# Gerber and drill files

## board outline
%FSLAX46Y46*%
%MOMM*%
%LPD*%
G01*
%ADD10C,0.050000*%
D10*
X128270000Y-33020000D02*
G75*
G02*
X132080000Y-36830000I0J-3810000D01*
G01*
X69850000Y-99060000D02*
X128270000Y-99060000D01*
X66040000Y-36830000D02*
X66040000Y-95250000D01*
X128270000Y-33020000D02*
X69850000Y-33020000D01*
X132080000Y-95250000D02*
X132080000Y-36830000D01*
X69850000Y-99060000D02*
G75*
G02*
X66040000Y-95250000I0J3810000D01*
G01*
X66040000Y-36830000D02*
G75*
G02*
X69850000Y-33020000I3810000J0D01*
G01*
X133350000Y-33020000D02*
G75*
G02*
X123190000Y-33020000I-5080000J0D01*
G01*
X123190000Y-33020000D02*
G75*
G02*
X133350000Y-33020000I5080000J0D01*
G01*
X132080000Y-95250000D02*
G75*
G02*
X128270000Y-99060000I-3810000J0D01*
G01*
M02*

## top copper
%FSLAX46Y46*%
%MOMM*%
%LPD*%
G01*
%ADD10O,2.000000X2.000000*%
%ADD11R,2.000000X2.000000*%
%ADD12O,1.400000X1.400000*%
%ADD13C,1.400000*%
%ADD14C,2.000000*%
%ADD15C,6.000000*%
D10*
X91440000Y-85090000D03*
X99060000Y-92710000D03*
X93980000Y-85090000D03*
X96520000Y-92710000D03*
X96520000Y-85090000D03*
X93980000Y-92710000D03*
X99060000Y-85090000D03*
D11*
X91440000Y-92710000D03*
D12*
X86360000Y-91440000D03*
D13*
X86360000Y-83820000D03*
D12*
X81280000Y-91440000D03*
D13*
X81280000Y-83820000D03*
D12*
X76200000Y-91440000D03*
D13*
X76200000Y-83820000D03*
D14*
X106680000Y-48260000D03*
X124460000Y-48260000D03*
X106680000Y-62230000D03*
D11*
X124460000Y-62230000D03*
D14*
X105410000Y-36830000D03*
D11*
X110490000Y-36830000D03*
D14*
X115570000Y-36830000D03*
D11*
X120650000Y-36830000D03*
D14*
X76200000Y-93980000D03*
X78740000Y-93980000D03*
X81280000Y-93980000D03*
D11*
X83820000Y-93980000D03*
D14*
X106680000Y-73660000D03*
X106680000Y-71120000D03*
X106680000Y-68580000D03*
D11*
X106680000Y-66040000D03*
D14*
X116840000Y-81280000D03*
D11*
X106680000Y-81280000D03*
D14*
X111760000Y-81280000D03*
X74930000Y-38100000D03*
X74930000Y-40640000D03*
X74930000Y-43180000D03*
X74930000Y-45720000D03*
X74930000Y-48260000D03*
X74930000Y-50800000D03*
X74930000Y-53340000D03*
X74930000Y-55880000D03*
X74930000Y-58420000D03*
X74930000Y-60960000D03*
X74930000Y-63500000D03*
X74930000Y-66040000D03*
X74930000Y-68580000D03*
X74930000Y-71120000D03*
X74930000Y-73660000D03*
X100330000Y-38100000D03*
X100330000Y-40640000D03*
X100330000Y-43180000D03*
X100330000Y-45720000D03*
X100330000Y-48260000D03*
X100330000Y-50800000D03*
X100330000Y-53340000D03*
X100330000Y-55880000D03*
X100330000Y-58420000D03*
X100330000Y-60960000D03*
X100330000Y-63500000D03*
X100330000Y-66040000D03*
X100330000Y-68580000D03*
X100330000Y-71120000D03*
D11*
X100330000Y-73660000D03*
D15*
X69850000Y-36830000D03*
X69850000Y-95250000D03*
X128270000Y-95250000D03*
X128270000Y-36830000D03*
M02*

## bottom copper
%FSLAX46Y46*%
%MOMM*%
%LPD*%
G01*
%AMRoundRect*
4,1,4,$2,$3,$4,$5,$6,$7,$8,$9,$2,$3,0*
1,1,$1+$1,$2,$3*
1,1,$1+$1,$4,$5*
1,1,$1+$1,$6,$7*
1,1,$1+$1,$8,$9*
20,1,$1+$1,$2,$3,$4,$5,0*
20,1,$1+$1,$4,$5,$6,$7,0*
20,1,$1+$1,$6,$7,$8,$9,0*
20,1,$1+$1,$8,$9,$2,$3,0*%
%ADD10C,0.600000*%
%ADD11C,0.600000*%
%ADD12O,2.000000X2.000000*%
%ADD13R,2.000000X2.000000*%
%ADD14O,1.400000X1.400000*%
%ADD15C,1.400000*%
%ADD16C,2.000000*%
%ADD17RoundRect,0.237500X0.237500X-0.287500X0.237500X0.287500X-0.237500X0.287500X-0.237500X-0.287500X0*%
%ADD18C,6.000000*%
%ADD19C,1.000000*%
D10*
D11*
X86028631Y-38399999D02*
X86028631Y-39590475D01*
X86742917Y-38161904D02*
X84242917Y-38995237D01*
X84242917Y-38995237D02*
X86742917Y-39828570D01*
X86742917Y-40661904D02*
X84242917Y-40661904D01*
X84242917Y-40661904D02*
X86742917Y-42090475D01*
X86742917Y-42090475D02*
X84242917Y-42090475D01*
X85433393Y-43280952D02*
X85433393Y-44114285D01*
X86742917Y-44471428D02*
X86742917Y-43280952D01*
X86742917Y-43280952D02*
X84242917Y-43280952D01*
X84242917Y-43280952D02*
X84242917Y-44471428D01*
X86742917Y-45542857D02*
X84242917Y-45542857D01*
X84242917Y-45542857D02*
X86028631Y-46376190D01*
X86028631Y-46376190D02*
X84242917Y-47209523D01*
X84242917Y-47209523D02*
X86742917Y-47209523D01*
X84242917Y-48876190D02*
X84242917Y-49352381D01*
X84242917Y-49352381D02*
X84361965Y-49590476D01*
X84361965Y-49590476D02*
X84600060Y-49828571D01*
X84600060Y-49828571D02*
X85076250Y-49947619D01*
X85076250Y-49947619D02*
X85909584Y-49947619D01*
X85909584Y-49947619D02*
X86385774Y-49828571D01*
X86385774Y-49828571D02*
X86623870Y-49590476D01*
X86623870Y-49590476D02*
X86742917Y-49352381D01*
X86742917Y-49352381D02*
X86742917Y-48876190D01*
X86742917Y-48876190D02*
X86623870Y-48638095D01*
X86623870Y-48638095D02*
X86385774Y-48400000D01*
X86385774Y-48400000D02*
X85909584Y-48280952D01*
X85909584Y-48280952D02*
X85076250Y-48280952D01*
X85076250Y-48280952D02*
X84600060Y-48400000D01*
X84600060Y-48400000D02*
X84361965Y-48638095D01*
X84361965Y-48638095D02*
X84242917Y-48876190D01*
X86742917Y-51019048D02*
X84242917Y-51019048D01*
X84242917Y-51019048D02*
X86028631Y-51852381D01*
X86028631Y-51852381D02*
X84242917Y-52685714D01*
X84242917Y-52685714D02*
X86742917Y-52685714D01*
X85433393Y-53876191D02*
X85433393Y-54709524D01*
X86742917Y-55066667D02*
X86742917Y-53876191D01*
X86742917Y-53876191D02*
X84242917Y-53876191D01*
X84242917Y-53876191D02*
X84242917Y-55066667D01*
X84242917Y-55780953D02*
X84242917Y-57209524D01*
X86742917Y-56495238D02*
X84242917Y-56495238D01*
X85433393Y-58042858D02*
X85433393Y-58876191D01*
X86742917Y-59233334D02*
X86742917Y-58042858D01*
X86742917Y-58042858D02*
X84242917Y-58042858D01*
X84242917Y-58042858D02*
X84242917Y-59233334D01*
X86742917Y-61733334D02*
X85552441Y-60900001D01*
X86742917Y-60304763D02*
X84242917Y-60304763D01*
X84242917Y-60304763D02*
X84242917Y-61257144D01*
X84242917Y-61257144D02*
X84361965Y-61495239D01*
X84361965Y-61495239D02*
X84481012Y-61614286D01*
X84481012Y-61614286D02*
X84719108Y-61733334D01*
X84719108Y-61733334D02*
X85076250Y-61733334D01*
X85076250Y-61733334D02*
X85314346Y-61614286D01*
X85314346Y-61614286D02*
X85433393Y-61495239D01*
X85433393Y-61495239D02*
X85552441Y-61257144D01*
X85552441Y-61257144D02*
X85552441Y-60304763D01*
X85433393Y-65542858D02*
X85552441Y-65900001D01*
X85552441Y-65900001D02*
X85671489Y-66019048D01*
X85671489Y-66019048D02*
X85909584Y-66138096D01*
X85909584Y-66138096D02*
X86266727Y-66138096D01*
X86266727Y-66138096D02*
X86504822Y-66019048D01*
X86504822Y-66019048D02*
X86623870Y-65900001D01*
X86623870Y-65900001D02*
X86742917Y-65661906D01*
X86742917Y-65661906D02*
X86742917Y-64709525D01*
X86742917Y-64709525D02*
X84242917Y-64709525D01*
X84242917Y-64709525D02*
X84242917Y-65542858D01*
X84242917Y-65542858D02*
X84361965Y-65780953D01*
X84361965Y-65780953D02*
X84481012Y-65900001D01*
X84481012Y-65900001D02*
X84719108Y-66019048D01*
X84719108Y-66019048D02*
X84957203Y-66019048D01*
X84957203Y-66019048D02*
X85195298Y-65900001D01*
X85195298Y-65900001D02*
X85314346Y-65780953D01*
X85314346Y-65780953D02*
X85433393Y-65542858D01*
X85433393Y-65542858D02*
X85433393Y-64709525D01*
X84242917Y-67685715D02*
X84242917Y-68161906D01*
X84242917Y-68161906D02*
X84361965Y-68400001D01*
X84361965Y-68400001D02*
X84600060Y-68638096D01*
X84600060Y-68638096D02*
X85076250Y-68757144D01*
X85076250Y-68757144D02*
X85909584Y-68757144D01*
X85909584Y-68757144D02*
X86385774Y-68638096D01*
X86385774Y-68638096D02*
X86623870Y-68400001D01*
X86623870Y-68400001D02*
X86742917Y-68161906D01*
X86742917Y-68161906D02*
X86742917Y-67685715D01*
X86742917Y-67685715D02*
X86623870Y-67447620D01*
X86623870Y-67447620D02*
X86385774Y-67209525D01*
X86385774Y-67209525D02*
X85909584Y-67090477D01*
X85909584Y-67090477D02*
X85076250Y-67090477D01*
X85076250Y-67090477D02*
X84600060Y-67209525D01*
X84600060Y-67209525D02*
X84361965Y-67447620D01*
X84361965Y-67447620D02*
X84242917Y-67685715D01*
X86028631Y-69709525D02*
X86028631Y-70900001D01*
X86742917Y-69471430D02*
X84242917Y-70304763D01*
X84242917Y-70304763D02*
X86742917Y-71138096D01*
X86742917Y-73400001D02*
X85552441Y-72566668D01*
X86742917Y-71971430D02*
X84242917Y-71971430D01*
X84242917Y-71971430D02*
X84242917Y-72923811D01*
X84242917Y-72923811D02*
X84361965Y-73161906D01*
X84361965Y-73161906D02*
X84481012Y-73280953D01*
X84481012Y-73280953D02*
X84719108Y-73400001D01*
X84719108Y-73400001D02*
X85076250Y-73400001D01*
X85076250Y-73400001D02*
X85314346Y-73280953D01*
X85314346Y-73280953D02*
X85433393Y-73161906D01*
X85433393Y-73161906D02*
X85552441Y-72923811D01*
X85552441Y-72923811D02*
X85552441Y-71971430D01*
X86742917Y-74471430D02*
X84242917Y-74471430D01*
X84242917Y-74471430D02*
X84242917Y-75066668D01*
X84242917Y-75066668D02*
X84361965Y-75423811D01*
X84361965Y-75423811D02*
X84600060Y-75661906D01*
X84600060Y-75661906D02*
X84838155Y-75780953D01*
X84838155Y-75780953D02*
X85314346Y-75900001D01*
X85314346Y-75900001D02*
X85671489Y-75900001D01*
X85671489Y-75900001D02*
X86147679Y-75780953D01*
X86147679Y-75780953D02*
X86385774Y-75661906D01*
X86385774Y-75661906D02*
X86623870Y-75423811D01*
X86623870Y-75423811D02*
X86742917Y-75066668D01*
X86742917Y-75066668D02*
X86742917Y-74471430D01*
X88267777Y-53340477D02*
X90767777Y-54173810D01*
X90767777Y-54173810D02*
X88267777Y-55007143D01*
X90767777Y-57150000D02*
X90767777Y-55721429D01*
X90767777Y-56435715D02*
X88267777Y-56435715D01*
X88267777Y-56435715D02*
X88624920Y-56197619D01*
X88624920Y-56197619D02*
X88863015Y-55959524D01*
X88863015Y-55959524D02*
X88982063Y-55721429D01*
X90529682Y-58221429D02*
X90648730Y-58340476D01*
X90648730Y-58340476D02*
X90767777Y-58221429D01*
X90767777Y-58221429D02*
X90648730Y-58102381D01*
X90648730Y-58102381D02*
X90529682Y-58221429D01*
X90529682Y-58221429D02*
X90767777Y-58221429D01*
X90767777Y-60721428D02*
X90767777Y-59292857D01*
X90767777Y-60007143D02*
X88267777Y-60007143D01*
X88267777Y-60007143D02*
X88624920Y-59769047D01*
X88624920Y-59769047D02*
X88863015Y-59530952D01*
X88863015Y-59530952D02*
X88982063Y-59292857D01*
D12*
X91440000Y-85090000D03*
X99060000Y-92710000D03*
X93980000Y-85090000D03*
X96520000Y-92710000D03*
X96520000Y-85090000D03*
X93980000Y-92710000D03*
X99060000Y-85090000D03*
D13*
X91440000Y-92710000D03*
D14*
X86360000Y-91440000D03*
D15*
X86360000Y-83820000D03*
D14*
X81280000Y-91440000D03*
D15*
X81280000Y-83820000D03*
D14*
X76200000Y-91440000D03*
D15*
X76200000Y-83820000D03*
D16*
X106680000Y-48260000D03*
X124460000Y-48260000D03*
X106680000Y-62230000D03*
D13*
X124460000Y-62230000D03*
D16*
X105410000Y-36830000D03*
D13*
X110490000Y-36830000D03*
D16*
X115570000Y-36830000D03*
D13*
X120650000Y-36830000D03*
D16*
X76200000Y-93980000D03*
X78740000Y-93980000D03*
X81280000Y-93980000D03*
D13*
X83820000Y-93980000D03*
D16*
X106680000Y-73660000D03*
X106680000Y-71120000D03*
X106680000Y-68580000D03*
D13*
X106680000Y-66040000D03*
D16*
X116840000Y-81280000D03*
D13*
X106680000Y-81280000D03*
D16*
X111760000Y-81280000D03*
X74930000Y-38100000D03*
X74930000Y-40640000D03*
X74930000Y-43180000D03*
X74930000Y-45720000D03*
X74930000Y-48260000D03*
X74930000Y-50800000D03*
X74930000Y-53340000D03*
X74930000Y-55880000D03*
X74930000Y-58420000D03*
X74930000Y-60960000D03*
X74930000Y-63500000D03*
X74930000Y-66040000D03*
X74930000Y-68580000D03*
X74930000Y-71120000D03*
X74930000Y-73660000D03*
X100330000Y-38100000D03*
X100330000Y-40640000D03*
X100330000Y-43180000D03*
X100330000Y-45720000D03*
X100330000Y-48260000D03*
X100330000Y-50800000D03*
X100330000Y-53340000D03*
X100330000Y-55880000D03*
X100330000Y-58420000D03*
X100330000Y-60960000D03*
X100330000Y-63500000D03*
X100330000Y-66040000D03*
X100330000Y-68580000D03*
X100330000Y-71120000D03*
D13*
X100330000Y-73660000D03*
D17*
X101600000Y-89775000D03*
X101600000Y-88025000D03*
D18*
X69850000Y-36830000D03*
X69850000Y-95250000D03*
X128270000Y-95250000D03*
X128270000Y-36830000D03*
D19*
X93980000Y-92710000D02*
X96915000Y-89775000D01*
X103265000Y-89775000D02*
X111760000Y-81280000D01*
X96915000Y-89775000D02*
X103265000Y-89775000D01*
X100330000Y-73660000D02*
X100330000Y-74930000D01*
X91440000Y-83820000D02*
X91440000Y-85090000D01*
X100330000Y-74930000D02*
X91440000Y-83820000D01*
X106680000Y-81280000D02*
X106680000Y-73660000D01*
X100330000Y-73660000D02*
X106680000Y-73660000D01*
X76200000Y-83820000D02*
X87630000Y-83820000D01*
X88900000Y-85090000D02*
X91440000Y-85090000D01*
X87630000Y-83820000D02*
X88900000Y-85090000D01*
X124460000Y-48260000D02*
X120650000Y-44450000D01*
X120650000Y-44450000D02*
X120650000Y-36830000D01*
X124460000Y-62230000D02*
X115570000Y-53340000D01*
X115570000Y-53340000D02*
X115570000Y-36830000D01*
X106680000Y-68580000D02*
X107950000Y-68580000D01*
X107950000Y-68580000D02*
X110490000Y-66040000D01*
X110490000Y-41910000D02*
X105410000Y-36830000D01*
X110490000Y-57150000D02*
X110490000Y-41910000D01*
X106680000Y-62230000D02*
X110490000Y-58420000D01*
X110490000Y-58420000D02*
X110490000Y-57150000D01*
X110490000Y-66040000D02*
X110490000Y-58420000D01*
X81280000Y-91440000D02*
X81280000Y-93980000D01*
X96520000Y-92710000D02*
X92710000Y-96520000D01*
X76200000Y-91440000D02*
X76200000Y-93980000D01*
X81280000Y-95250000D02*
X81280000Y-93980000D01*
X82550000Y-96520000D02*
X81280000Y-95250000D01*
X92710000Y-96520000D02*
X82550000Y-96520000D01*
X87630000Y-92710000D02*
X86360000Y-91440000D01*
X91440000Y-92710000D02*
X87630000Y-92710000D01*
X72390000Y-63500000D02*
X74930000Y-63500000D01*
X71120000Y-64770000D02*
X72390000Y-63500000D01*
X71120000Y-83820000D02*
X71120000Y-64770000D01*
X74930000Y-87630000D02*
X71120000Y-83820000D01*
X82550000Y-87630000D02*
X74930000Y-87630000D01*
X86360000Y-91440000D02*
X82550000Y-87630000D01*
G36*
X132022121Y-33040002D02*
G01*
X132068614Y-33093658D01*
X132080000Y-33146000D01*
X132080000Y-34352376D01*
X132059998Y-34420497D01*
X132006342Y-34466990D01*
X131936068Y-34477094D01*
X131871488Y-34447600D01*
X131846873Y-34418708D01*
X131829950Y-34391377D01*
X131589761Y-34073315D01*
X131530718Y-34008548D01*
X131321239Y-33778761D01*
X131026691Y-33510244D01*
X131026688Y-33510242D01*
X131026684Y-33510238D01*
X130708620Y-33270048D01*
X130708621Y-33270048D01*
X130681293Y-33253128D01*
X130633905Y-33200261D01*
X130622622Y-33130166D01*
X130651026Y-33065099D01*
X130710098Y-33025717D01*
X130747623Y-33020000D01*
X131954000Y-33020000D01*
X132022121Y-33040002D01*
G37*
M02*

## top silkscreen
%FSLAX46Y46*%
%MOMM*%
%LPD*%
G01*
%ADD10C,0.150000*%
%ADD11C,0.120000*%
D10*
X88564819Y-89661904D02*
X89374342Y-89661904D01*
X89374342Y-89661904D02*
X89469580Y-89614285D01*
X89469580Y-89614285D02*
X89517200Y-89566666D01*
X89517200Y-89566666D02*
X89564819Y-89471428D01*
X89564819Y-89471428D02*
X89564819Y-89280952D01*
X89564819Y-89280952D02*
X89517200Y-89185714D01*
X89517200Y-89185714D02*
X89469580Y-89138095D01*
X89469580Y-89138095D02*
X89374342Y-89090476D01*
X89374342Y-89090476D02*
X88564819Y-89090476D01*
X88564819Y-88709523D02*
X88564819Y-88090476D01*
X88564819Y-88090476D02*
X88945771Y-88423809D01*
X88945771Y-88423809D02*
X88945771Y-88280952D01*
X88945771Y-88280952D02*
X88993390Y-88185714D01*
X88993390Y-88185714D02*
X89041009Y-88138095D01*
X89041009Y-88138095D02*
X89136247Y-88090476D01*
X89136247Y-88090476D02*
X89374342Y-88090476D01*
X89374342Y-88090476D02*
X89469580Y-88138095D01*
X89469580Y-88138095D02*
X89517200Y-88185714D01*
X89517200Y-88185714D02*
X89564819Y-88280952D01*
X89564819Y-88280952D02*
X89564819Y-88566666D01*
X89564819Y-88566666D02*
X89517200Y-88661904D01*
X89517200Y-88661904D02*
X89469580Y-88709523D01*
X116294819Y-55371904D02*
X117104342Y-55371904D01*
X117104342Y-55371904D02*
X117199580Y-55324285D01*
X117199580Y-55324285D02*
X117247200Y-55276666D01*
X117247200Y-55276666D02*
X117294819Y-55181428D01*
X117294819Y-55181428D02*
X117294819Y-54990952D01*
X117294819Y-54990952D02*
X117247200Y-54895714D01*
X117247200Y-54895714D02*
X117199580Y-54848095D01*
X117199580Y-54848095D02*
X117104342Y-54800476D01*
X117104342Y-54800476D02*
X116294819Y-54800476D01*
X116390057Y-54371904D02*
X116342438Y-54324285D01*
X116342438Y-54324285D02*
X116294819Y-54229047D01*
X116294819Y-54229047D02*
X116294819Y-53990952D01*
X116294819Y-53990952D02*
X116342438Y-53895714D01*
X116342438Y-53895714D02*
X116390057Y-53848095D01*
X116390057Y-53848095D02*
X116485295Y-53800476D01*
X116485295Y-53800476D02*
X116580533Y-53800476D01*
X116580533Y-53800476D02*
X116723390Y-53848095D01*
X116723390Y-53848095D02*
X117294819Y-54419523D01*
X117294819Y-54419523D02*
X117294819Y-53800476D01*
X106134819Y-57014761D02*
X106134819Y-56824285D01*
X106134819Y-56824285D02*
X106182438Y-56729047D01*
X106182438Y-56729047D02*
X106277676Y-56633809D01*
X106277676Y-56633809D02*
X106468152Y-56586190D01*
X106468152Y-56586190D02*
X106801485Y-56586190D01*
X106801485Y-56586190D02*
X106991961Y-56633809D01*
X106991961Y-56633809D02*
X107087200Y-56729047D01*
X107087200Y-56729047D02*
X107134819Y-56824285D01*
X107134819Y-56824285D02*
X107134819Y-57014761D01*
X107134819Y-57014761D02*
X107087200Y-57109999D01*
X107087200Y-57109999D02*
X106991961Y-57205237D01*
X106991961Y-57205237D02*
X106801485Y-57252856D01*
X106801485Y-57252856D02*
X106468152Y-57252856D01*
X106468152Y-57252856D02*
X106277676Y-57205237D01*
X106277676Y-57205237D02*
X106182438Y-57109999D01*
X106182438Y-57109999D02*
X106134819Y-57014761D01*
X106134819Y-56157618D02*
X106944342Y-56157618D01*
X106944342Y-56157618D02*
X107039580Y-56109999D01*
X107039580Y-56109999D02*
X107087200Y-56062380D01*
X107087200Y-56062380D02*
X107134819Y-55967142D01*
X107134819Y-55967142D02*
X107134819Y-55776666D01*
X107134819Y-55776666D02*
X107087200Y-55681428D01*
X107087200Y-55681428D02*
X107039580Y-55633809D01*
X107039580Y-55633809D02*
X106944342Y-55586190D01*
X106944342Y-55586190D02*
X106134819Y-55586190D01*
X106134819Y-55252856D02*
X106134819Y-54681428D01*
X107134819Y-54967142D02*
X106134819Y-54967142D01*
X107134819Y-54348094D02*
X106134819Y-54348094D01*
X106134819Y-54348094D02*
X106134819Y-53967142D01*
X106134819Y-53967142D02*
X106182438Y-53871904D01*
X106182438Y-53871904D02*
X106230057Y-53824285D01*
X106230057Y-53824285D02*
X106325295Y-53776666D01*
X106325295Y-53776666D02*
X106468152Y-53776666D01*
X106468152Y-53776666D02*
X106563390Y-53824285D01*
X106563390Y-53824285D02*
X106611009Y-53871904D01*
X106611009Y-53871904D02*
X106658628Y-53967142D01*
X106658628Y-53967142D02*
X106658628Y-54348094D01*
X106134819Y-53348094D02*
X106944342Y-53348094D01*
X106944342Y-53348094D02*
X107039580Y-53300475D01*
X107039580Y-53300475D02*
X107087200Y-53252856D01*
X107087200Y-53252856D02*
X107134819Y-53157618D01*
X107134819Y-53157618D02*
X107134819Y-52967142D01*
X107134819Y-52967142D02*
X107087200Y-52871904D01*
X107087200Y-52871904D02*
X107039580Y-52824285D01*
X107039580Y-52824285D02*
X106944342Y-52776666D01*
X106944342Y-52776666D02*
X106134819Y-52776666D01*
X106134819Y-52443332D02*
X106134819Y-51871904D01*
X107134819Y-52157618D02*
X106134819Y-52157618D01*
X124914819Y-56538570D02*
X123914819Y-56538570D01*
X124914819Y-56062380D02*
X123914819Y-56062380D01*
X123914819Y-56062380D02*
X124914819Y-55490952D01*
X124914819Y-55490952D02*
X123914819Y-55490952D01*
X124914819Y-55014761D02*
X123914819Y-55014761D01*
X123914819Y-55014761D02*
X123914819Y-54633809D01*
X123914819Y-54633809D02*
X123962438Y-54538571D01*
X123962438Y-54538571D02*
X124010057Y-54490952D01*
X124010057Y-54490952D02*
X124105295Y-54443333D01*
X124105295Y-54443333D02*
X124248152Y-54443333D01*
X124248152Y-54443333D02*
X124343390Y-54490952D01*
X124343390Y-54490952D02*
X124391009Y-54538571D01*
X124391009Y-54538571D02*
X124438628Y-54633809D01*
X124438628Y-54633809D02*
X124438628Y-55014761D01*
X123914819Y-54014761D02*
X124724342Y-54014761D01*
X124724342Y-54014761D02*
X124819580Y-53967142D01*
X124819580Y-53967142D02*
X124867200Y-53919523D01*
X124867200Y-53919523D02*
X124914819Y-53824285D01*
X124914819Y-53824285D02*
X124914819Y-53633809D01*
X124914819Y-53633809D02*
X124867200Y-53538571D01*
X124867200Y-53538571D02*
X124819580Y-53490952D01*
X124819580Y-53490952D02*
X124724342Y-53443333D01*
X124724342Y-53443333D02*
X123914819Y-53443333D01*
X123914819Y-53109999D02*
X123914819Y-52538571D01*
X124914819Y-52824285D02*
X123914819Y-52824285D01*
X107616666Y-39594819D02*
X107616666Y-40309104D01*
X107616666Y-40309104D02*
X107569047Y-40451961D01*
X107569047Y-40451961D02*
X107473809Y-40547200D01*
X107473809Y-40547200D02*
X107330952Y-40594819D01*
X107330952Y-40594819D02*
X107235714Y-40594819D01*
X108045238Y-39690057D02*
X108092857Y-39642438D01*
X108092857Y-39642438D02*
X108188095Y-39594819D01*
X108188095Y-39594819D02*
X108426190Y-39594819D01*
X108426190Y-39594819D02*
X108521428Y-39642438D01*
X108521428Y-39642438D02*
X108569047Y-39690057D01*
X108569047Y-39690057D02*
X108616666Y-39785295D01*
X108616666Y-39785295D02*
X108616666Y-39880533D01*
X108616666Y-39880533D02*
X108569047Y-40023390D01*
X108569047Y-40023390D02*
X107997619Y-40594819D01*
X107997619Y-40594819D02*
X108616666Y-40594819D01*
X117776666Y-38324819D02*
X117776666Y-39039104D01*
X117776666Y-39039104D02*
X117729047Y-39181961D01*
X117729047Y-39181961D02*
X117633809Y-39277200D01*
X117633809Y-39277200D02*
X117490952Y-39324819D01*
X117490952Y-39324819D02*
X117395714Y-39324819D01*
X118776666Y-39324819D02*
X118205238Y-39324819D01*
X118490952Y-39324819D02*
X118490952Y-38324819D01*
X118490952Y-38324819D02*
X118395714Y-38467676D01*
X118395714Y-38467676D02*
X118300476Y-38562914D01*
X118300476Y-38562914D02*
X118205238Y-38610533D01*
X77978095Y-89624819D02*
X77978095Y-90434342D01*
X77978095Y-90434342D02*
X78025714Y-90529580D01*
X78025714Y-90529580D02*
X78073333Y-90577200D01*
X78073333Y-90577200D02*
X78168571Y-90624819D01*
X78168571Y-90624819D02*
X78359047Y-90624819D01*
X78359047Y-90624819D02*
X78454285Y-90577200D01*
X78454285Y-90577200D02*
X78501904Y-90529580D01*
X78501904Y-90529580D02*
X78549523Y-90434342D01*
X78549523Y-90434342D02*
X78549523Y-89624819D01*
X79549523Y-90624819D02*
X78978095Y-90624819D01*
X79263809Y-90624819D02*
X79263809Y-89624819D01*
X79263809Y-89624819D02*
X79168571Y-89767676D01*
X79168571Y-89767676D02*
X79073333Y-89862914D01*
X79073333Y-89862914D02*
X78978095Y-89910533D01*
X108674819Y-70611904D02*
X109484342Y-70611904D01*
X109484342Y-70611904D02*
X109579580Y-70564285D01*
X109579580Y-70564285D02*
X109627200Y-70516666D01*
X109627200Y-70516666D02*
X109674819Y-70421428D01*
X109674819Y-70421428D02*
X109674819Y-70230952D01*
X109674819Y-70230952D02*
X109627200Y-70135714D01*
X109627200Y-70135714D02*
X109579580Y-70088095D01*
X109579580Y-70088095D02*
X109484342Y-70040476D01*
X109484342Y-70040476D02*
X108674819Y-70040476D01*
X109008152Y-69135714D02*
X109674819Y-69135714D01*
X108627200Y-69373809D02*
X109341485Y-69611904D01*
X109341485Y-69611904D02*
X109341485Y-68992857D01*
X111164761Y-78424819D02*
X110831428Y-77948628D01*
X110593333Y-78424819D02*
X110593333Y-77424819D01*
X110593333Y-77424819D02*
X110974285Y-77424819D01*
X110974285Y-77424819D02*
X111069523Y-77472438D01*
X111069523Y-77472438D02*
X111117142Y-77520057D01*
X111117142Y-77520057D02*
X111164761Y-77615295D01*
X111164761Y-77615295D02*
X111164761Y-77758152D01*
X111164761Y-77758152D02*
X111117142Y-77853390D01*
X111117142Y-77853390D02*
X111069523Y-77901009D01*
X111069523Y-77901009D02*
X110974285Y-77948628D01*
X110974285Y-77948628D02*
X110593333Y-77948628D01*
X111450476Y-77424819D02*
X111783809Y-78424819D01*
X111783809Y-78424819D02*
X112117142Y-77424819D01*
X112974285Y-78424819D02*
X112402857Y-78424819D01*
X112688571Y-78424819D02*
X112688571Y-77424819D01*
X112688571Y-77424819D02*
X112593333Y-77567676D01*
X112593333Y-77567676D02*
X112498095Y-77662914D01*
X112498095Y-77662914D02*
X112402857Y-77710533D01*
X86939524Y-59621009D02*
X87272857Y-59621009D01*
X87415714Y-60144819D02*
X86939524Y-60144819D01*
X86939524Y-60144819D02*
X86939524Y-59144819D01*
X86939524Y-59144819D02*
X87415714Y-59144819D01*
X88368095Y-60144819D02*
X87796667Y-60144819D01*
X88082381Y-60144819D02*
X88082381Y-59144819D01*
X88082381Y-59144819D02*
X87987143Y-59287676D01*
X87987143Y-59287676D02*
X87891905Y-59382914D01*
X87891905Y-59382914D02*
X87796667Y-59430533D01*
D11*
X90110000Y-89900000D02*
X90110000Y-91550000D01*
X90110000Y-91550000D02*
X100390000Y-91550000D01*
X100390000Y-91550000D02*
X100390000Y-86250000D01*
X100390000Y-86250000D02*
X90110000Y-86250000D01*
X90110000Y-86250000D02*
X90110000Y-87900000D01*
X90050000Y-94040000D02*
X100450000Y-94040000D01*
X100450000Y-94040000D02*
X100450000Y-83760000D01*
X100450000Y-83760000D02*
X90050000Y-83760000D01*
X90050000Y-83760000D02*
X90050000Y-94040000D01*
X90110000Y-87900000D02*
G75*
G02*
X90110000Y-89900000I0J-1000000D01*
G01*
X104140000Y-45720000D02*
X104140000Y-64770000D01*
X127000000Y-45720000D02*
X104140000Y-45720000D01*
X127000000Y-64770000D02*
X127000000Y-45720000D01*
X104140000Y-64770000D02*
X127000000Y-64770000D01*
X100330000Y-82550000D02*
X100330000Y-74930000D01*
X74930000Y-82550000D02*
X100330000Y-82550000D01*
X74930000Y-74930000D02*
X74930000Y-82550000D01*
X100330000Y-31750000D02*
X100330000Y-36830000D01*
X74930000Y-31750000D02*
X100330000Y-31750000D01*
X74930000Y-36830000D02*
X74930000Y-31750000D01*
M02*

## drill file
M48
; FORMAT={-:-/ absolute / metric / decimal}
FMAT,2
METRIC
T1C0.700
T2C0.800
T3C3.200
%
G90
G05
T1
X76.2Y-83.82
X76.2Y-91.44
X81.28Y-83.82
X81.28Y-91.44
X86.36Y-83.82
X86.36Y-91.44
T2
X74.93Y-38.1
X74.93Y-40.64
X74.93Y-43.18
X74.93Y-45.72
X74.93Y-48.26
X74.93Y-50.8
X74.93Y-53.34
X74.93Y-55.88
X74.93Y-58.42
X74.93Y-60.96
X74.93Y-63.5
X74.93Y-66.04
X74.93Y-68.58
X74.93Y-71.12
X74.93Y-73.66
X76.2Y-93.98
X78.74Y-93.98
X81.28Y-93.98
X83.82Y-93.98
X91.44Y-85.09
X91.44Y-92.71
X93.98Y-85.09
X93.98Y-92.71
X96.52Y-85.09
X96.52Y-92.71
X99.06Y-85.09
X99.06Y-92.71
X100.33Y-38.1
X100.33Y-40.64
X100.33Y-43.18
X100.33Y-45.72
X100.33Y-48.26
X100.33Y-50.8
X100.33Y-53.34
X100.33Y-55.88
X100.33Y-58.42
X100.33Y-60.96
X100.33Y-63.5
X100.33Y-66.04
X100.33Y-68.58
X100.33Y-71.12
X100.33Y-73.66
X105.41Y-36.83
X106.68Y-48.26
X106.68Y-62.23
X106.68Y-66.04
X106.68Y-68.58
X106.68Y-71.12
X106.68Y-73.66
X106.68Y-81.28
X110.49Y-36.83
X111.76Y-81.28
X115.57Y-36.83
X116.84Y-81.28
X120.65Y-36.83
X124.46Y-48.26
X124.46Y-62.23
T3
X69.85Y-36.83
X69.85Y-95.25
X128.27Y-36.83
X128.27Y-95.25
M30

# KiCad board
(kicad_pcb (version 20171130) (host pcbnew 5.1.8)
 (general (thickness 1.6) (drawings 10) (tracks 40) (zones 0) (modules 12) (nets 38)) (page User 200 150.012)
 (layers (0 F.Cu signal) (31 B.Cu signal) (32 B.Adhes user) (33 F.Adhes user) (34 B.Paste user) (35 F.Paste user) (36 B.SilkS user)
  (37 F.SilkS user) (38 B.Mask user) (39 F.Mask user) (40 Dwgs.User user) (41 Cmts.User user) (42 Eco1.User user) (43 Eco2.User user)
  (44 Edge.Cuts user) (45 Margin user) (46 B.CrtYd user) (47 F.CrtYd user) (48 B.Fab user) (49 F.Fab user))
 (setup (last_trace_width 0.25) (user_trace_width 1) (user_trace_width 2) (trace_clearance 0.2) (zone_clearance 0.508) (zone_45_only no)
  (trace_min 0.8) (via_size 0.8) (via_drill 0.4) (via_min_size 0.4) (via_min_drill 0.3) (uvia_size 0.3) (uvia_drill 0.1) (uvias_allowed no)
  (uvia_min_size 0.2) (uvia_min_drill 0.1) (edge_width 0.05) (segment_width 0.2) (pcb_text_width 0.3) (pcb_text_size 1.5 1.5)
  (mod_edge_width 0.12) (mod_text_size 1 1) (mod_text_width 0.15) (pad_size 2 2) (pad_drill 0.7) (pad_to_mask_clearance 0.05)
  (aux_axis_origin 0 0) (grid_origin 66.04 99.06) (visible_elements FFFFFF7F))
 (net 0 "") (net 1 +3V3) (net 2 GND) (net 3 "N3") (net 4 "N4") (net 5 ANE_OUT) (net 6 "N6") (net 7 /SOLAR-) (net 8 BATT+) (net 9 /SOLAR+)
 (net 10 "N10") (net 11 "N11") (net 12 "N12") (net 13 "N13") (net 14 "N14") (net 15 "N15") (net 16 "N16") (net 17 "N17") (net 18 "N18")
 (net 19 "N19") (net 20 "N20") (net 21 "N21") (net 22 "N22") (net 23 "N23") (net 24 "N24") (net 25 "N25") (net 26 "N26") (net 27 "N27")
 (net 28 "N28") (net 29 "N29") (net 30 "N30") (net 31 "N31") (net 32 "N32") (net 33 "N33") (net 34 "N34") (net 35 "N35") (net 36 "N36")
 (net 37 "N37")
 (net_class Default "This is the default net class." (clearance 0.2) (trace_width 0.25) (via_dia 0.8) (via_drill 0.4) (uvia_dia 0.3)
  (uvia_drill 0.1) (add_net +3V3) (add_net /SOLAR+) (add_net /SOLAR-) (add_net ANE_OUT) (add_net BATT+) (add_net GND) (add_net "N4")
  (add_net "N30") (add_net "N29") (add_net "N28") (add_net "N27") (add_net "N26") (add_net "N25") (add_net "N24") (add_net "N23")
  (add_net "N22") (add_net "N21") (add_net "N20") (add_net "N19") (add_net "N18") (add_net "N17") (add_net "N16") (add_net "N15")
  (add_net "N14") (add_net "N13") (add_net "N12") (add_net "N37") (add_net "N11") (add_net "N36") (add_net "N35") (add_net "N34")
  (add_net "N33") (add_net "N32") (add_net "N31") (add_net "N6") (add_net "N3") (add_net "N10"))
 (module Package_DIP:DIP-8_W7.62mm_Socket (layer F.Cu) (at 91.44 92.71 90)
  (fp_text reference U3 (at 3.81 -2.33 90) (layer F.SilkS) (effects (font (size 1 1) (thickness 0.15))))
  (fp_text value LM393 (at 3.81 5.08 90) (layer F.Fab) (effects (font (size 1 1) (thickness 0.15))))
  (fp_line (start 2.81 -1.33) (end 1.16 -1.33) (layer F.SilkS) (width 0.12))
  (fp_line (start 1.16 -1.33) (end 1.16 8.95) (layer F.SilkS) (width 0.12))
  (fp_line (start 1.16 8.95) (end 6.46 8.95) (layer F.SilkS) (width 0.12))
  (fp_line (start 6.46 8.95) (end 6.46 -1.33) (layer F.SilkS) (width 0.12))
  (fp_line (start 6.46 -1.33) (end 4.81 -1.33) (layer F.SilkS) (width 0.12))
  (fp_line (start -1.33 -1.39) (end -1.33 9.01) (layer F.SilkS) (width 0.12))
  (fp_line (start -1.33 9.01) (end 8.95 9.01) (layer F.SilkS) (width 0.12))
  (fp_line (start 8.95 9.01) (end 8.95 -1.39) (layer F.SilkS) (width 0.12))
  (fp_line (start 8.95 -1.39) (end -1.33 -1.39) (layer F.SilkS) (width 0.12))
  (fp_arc (start 3.81 -1.33) (end 2.81 -1.33) (angle -180) (layer F.SilkS) (width 0.12))
  (pad 8 thru_hole oval (at 7.62 0 90) (size 2 2) (drill 0.8) (layers *.Cu *.Mask) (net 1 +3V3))
  (pad 4 thru_hole oval (at 0 7.62 90) (size 2 2) (drill 0.8) (layers *.Cu *.Mask) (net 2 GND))
  (pad 7 thru_hole oval (at 7.62 2.54 90) (size 2 2) (drill 0.8) (layers *.Cu *.Mask))
  (pad 3 thru_hole oval (at 0 5.08 90) (size 2 2) (drill 0.8) (layers *.Cu *.Mask) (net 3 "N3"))
  (pad 6 thru_hole oval (at 7.62 5.08 90) (size 2 2) (drill 0.8) (layers *.Cu *.Mask))
  (pad 2 thru_hole oval (at 0 2.54 90) (size 2 2) (drill 0.8) (layers *.Cu *.Mask) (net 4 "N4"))
  (pad 5 thru_hole oval (at 7.62 7.62 90) (size 2 2) (drill 0.8) (layers *.Cu *.Mask))
  (pad 1 thru_hole rect (at 0 0 90) (size 2 2) (drill 0.8) (layers *.Cu *.Mask) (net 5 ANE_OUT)))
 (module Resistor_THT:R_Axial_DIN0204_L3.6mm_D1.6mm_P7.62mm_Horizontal (layer B.Cu) (at 86.36 83.82 270)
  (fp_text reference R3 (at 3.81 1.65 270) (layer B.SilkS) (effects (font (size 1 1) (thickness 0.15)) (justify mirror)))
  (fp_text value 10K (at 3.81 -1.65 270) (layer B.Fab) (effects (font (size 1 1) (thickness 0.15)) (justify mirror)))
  (pad 2 thru_hole oval (at 7.62 0 270) (size 1.4 1.4) (drill 0.7) (layers *.Cu *.Mask) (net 5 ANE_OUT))
  (pad 1 thru_hole circle (at 0 0 270) (size 1.4 1.4) (drill 0.7) (layers *.Cu *.Mask) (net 1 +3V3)))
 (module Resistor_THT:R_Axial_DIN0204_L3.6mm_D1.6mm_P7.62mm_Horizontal (layer B.Cu) (at 81.28 83.82 270)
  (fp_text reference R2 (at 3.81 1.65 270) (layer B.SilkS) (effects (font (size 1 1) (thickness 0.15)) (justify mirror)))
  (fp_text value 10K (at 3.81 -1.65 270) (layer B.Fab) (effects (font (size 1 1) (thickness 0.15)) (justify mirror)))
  (pad 2 thru_hole oval (at 7.62 0 270) (size 1.4 1.4) (drill 0.7) (layers *.Cu *.Mask) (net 3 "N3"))
  (pad 1 thru_hole circle (at 0 0 270) (size 1.4 1.4) (drill 0.7) (layers *.Cu *.Mask) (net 1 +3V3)))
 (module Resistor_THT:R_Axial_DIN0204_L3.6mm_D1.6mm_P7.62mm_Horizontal (layer B.Cu) (at 76.2 83.82 270)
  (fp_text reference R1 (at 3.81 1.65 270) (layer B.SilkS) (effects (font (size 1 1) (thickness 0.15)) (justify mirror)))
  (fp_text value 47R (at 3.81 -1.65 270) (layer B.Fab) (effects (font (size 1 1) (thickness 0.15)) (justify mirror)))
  (pad 2 thru_hole oval (at 7.62 0 270) (size 1.4 1.4) (drill 0.7) (layers *.Cu *.Mask) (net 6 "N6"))
  (pad 1 thru_hole circle (at 0 0 270) (size 1.4 1.4) (drill 0.7) (layers *.Cu *.Mask) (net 1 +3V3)))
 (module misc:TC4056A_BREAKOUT (layer F.Cu) (at 115.57 54.61 90)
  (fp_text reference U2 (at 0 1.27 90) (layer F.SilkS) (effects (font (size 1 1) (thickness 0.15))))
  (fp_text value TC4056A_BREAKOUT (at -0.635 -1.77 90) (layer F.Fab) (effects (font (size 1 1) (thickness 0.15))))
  (fp_line (start 8.89 -11.43) (end -10.16 -11.43) (layer F.SilkS) (width 0.12))
  (fp_line (start 8.89 11.43) (end 8.89 -11.43) (layer F.SilkS) (width 0.12))
  (fp_line (start -10.16 11.43) (end 8.89 11.43) (layer F.SilkS) (width 0.12))
  (fp_line (start -10.16 -11.43) (end -10.16 11.43) (layer F.SilkS) (width 0.12))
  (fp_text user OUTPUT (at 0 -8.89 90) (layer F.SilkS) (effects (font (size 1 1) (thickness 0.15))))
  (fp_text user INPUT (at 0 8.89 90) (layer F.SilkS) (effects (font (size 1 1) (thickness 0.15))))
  (pad 3 thru_hole circle (at 6.35 -8.89 90) (size 2 2) (drill 0.8) (layers *.Cu *.Mask) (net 2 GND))
  (pad 2 thru_hole circle (at 6.35 8.89 90) (size 2 2) (drill 0.8) (layers *.Cu *.Mask) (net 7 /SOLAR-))
  (pad 4 thru_hole circle (at -7.62 -8.89 90) (size 2 2) (drill 0.8) (layers *.Cu *.Mask) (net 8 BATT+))
  (pad 1 thru_hole rect (at -7.62 8.89 90) (size 2 2) (drill 0.8) (layers *.Cu *.Mask) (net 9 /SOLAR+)))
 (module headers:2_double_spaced (layer F.Cu) (at 107.95 36.83 180)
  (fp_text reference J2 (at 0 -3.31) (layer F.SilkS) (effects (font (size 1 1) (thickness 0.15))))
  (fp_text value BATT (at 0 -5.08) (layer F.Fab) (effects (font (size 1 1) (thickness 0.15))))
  (pad 2 thru_hole circle (at 2.54 0 180) (size 2 2) (drill 0.8) (layers *.Cu *.Mask) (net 8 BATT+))
  (pad 1 thru_hole rect (at -2.54 0 180) (size 2 2) (drill 0.8) (layers *.Cu *.Mask) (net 2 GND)))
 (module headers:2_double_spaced (layer F.Cu) (at 118.11 36.83 180)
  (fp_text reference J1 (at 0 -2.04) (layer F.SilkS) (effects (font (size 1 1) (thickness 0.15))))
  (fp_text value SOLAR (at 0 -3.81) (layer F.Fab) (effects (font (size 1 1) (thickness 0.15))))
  (pad 2 thru_hole circle (at 2.54 0 180) (size 2 2) (drill 0.8) (layers *.Cu *.Mask) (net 9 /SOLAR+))
  (pad 1 thru_hole rect (at -2.54 0 180) (size 2 2) (drill 0.8) (layers *.Cu *.Mask) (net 7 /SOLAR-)))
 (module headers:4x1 (layer F.Cu) (at 80.01 93.98 180)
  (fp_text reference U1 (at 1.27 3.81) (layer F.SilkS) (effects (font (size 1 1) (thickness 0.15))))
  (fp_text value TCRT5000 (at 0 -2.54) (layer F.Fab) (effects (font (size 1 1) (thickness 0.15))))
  (pad 4 thru_hole circle (at 3.81 0 180) (size 2 2) (drill 0.8) (layers *.Cu *.Mask) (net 6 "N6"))
  (pad 3 thru_hole circle (at 1.27 0 180) (size 2 2) (drill 0.8) (layers *.Cu *.Mask) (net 2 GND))
  (pad 2 thru_hole circle (at -1.27 0 180) (size 2 2) (drill 0.8) (layers *.Cu *.Mask) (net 3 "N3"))
  (pad 1 thru_hole rect (at -3.81 0 180) (size 2 2) (drill 0.8) (layers *.Cu *.Mask) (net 2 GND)))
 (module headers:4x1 (layer F.Cu) (at 106.68 69.85 270)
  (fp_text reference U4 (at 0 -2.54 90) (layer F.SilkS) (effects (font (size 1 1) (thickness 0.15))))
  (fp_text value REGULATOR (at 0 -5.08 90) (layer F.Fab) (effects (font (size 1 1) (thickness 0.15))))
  (pad 4 thru_hole circle (at 3.81 0 270) (size 2 2) (drill 0.8) (layers *.Cu *.Mask) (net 1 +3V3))
  (pad 3 thru_hole circle (at 1.27 0 270) (size 2 2) (drill 0.8) (layers *.Cu *.Mask) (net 2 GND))
  (pad 2 thru_hole circle (at -1.27 0 270) (size 2 2) (drill 0.8) (layers *.Cu *.Mask) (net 8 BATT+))
  (pad 1 thru_hole rect (at -3.81 0 270) (size 2 2) (drill 0.8) (layers *.Cu *.Mask) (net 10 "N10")))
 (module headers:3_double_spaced (layer F.Cu) (at 111.76 81.28)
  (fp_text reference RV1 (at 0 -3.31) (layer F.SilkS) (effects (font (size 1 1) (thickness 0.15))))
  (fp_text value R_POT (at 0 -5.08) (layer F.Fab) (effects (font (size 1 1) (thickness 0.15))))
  (pad 3 thru_hole circle (at 5.08 0) (size 2 2) (drill 0.8) (layers *.Cu *.Mask) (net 2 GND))
  (pad 1 thru_hole rect (at -5.08 0) (size 2 2) (drill 0.8) (layers *.Cu *.Mask) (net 1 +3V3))
  (pad 2 thru_hole circle (at 0 0) (size 2 2) (drill 0.8) (layers *.Cu *.Mask) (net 4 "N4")))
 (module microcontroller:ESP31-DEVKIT (layer F.Cu) (at 87.63 57.15)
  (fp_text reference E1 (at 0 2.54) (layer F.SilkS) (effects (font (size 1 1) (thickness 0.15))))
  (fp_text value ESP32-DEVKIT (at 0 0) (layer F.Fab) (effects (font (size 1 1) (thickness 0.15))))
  (fp_line (start 12.7 25.4) (end 12.7 17.78) (layer F.SilkS) (width 0.12))
  (fp_line (start -12.7 25.4) (end 12.7 25.4) (layer F.SilkS) (width 0.12))
  (fp_line (start -12.7 17.78) (end -12.7 25.4) (layer F.SilkS) (width 0.12))
  (fp_line (start 12.7 -25.4) (end 12.7 -20.32) (layer F.SilkS) (width 0.12))
  (fp_line (start -12.7 -25.4) (end 12.7 -25.4) (layer F.SilkS) (width 0.12))
  (fp_line (start -12.7 -20.32) (end -12.7 -25.4) (layer F.SilkS) (width 0.12))
  (pad 30 thru_hole circle (at -12.7 -19.05) (size 2 2) (drill 0.8) (layers *.Cu *.Mask) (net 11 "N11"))
  (pad 29 thru_hole circle (at -12.7 -16.51) (size 2 2) (drill 0.8) (layers *.Cu *.Mask) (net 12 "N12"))
  (pad 28 thru_hole circle (at -12.7 -13.97) (size 2 2) (drill 0.8) (layers *.Cu *.Mask) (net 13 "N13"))
  (pad 27 thru_hole circle (at -12.7 -11.43) (size 2 2) (drill 0.8) (layers *.Cu *.Mask) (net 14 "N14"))
  (pad 26 thru_hole circle (at -12.7 -8.89) (size 2 2) (drill 0.8) (layers *.Cu *.Mask) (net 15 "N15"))
  (pad 25 thru_hole circle (at -12.7 -6.35) (size 2 2) (drill 0.8) (layers *.Cu *.Mask) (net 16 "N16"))
  (pad 24 thru_hole circle (at -12.7 -3.81) (size 2 2) (drill 0.8) (layers *.Cu *.Mask) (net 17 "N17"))
  (pad 23 thru_hole circle (at -12.7 -1.27) (size 2 2) (drill 0.8) (layers *.Cu *.Mask) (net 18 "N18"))
  (pad 22 thru_hole circle (at -12.7 1.27) (size 2 2) (drill 0.8) (layers *.Cu *.Mask) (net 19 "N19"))
  (pad 21 thru_hole circle (at -12.7 3.81) (size 2 2) (drill 0.8) (layers *.Cu *.Mask) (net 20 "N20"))
  (pad 20 thru_hole circle (at -12.7 6.35) (size 2 2) (drill 0.8) (layers *.Cu *.Mask) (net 5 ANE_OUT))
  (pad 19 thru_hole circle (at -12.7 8.89) (size 2 2) (drill 0.8) (layers *.Cu *.Mask) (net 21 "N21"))
  (pad 18 thru_hole circle (at -12.7 11.43) (size 2 2) (drill 0.8) (layers *.Cu *.Mask) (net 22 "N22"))
  (pad 17 thru_hole circle (at -12.7 13.97) (size 2 2) (drill 0.8) (layers *.Cu *.Mask) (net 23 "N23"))
  (pad 16 thru_hole circle (at -12.7 16.51) (size 2 2) (drill 0.8) (layers *.Cu *.Mask) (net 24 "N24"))
  (pad 15 thru_hole circle (at 12.7 -19.05) (size 2 2) (drill 0.8) (layers *.Cu *.Mask) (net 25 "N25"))
  (pad 14 thru_hole circle (at 12.7 -16.51) (size 2 2) (drill 0.8) (layers *.Cu *.Mask) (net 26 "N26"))
  (pad 13 thru_hole circle (at 12.7 -13.97) (size 2 2) (drill 0.8) (layers *.Cu *.Mask) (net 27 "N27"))
  (pad 12 thru_hole circle (at 12.7 -11.43) (size 2 2) (drill 0.8) (layers *.Cu *.Mask) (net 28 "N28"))
  (pad 11 thru_hole circle (at 12.7 -8.89) (size 2 2) (drill 0.8) (layers *.Cu *.Mask) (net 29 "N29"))
  (pad 10 thru_hole circle (at 12.7 -6.35) (size 2 2) (drill 0.8) (layers *.Cu *.Mask) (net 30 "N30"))
  (pad 9 thru_hole circle (at 12.7 -3.81) (size 2 2) (drill 0.8) (layers *.Cu *.Mask) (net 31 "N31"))
  (pad 8 thru_hole circle (at 12.7 -1.27) (size 2 2) (drill 0.8) (layers *.Cu *.Mask) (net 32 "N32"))
  (pad 7 thru_hole circle (at 12.7 1.27) (size 2 2) (drill 0.8) (layers *.Cu *.Mask) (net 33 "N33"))
  (pad 6 thru_hole circle (at 12.7 3.81) (size 2 2) (drill 0.8) (layers *.Cu *.Mask) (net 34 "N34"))
  (pad 5 thru_hole circle (at 12.7 6.35) (size 2 2) (drill 0.8) (layers *.Cu *.Mask) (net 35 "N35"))
  (pad 4 thru_hole circle (at 12.7 8.89) (size 2 2) (drill 0.8) (layers *.Cu *.Mask) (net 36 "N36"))
  (pad 3 thru_hole circle (at 12.7 11.43) (size 2 2) (drill 0.8) (layers *.Cu *.Mask) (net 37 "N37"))
  (pad 2 thru_hole circle (at 12.7 13.97) (size 2 2) (drill 0.8) (layers *.Cu *.Mask) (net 2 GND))
  (pad 1 thru_hole rect (at 12.7 16.51) (size 2 2) (drill 0.8) (layers *.Cu *.Mask) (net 1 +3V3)))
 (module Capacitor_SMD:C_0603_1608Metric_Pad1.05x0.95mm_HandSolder (layer B.Cu) (at 101.6 88.9 90)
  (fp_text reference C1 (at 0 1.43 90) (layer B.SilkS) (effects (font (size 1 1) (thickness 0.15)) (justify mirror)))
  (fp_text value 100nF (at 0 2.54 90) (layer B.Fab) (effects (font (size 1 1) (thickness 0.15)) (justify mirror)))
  (pad 1 smd roundrect (at -0.875 0 90) (size 1.05 0.95) (layers B.Cu B.Paste B.Mask) (roundrect_rratio 0.25) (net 4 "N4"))
  (pad 2 smd roundrect (at 0.875 0 90) (size 1.05 0.95) (layers B.Cu B.Paste B.Mask) (roundrect_rratio 0.25) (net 2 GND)))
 (gr_arc (start 128.27 36.83) (end 132.08 36.83) (angle -90) (layer Edge.Cuts) (width 0.05))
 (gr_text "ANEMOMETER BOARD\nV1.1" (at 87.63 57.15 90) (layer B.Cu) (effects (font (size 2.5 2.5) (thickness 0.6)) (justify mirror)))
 (gr_line (start 69.85 99.06) (end 128.27 99.06) (layer Edge.Cuts) (width 0.05))
 (gr_line (start 66.04 36.83) (end 66.04 95.25) (layer Edge.Cuts) (width 0.05))
 (gr_line (start 128.27 33.02) (end 69.85 33.02) (layer Edge.Cuts) (width 0.05))
 (gr_line (start 132.08 95.25) (end 132.08 36.83) (layer Edge.Cuts) (width 0.05))
 (gr_arc (start 69.85 95.25) (end 66.04 95.25) (angle -90) (layer Edge.Cuts) (width 0.05))
 (gr_arc (start 69.85 36.83) (end 69.85 33.02) (angle -90) (layer Edge.Cuts) (width 0.05))
 (gr_arc (start 128.27 33.02) (end 133.35 33.02) (angle 0) (layer Edge.Cuts) (width 0.05))
 (gr_arc (start 128.27 95.25) (end 128.27 99.06) (angle -90) (layer Edge.Cuts) (width 0.05))
 (via (at 69.85 36.83) (size 6) (drill 3.2) (layers F.Cu B.Cu) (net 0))
 (via (at 69.85 95.25) (size 6) (drill 3.2) (layers F.Cu B.Cu) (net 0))
 (via (at 128.27 95.25) (size 6) (drill 3.2) (layers F.Cu B.Cu) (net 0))
 (via (at 128.27 36.83) (size 6) (drill 3.2) (layers F.Cu B.Cu) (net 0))
 (segment (start 93.98 92.71) (end 96.915 89.775) (width 1) (layer B.Cu) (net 4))
 (segment (start 103.265 89.775) (end 111.76 81.28) (width 1) (layer B.Cu) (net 4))
 (segment (start 96.915 89.775) (end 103.265 89.775) (width 1) (layer B.Cu) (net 4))
 (segment (start 100.33 73.66) (end 100.33 74.93) (width 1) (layer B.Cu) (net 1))
 (segment (start 91.44 83.82) (end 91.44 85.09) (width 1) (layer B.Cu) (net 1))
 (segment (start 100.33 74.93) (end 91.44 83.82) (width 1) (layer B.Cu) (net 1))
 (segment (start 106.68 81.28) (end 106.68 73.66) (width 1) (layer B.Cu) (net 1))
 (segment (start 100.33 73.66) (end 106.68 73.66) (width 1) (layer B.Cu) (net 1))
 (segment (start 76.2 83.82) (end 87.63 83.82) (width 1) (layer B.Cu) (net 1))
 (segment (start 88.9 85.09) (end 91.44 85.09) (width 1) (layer B.Cu) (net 1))
 (segment (start 87.63 83.82) (end 88.9 85.09) (width 1) (layer B.Cu) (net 1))
 (segment (start 124.46 48.26) (end 120.65 44.45) (width 1) (layer B.Cu) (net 7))
 (segment (start 120.65 44.45) (end 120.65 36.83) (width 1) (layer B.Cu) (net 7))
 (segment (start 124.46 62.23) (end 115.57 53.34) (width 1) (layer B.Cu) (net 9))
 (segment (start 115.57 53.34) (end 115.57 36.83) (width 1) (layer B.Cu) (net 9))
 (segment (start 106.68 68.58) (end 107.95 68.58) (width 1) (layer B.Cu) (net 8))
 (segment (start 107.95 68.58) (end 110.49 66.04) (width 1) (layer B.Cu) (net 8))
 (segment (start 110.49 41.91) (end 105.41 36.83) (width 1) (layer B.Cu) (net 8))
 (segment (start 110.49 57.15) (end 110.49 41.91) (width 1) (layer B.Cu) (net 8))
 (segment (start 106.68 62.23) (end 110.49 58.42) (width 1) (layer B.Cu) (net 8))
 (segment (start 110.49 58.42) (end 110.49 57.15) (width 1) (layer B.Cu) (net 8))
 (segment (start 110.49 66.04) (end 110.49 58.42) (width 1) (layer B.Cu) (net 8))
 (segment (start 81.28 91.44) (end 81.28 93.98) (width 1) (layer B.Cu) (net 3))
 (segment (start 96.52 92.71) (end 92.71 96.52) (width 1) (layer B.Cu) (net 3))
 (segment (start 76.2 91.44) (end 76.2 93.98) (width 1) (layer B.Cu) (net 6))
 (segment (start 81.28 95.25) (end 81.28 93.98) (width 1) (layer B.Cu) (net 3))
 (segment (start 82.55 96.52) (end 81.28 95.25) (width 1) (layer B.Cu) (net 3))
 (segment (start 92.71 96.52) (end 82.55 96.52) (width 1) (layer B.Cu) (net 3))
 (segment (start 87.63 92.71) (end 86.36 91.44) (width 1) (layer B.Cu) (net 5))
 (segment (start 91.44 92.71) (end 87.63 92.71) (width 1) (layer B.Cu) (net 5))
 (segment (start 72.39 63.5) (end 74.93 63.5) (width 1) (layer B.Cu) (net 5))
 (segment (start 71.12 64.77) (end 72.39 63.5) (width 1) (layer B.Cu) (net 5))
 (segment (start 71.12 83.82) (end 71.12 64.77) (width 1) (layer B.Cu) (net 5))
 (segment (start 74.93 87.63) (end 71.12 83.82) (width 1) (layer B.Cu) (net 5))
 (segment (start 82.55 87.63) (end 74.93 87.63) (width 1) (layer B.Cu) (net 5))
 (segment (start 86.36 91.44) (end 82.55 87.63) (width 1) (layer B.Cu) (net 5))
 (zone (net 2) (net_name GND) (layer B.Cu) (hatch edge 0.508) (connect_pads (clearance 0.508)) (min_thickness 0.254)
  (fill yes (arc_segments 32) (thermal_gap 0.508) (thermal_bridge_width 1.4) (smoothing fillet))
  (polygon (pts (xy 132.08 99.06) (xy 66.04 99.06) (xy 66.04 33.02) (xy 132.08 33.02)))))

